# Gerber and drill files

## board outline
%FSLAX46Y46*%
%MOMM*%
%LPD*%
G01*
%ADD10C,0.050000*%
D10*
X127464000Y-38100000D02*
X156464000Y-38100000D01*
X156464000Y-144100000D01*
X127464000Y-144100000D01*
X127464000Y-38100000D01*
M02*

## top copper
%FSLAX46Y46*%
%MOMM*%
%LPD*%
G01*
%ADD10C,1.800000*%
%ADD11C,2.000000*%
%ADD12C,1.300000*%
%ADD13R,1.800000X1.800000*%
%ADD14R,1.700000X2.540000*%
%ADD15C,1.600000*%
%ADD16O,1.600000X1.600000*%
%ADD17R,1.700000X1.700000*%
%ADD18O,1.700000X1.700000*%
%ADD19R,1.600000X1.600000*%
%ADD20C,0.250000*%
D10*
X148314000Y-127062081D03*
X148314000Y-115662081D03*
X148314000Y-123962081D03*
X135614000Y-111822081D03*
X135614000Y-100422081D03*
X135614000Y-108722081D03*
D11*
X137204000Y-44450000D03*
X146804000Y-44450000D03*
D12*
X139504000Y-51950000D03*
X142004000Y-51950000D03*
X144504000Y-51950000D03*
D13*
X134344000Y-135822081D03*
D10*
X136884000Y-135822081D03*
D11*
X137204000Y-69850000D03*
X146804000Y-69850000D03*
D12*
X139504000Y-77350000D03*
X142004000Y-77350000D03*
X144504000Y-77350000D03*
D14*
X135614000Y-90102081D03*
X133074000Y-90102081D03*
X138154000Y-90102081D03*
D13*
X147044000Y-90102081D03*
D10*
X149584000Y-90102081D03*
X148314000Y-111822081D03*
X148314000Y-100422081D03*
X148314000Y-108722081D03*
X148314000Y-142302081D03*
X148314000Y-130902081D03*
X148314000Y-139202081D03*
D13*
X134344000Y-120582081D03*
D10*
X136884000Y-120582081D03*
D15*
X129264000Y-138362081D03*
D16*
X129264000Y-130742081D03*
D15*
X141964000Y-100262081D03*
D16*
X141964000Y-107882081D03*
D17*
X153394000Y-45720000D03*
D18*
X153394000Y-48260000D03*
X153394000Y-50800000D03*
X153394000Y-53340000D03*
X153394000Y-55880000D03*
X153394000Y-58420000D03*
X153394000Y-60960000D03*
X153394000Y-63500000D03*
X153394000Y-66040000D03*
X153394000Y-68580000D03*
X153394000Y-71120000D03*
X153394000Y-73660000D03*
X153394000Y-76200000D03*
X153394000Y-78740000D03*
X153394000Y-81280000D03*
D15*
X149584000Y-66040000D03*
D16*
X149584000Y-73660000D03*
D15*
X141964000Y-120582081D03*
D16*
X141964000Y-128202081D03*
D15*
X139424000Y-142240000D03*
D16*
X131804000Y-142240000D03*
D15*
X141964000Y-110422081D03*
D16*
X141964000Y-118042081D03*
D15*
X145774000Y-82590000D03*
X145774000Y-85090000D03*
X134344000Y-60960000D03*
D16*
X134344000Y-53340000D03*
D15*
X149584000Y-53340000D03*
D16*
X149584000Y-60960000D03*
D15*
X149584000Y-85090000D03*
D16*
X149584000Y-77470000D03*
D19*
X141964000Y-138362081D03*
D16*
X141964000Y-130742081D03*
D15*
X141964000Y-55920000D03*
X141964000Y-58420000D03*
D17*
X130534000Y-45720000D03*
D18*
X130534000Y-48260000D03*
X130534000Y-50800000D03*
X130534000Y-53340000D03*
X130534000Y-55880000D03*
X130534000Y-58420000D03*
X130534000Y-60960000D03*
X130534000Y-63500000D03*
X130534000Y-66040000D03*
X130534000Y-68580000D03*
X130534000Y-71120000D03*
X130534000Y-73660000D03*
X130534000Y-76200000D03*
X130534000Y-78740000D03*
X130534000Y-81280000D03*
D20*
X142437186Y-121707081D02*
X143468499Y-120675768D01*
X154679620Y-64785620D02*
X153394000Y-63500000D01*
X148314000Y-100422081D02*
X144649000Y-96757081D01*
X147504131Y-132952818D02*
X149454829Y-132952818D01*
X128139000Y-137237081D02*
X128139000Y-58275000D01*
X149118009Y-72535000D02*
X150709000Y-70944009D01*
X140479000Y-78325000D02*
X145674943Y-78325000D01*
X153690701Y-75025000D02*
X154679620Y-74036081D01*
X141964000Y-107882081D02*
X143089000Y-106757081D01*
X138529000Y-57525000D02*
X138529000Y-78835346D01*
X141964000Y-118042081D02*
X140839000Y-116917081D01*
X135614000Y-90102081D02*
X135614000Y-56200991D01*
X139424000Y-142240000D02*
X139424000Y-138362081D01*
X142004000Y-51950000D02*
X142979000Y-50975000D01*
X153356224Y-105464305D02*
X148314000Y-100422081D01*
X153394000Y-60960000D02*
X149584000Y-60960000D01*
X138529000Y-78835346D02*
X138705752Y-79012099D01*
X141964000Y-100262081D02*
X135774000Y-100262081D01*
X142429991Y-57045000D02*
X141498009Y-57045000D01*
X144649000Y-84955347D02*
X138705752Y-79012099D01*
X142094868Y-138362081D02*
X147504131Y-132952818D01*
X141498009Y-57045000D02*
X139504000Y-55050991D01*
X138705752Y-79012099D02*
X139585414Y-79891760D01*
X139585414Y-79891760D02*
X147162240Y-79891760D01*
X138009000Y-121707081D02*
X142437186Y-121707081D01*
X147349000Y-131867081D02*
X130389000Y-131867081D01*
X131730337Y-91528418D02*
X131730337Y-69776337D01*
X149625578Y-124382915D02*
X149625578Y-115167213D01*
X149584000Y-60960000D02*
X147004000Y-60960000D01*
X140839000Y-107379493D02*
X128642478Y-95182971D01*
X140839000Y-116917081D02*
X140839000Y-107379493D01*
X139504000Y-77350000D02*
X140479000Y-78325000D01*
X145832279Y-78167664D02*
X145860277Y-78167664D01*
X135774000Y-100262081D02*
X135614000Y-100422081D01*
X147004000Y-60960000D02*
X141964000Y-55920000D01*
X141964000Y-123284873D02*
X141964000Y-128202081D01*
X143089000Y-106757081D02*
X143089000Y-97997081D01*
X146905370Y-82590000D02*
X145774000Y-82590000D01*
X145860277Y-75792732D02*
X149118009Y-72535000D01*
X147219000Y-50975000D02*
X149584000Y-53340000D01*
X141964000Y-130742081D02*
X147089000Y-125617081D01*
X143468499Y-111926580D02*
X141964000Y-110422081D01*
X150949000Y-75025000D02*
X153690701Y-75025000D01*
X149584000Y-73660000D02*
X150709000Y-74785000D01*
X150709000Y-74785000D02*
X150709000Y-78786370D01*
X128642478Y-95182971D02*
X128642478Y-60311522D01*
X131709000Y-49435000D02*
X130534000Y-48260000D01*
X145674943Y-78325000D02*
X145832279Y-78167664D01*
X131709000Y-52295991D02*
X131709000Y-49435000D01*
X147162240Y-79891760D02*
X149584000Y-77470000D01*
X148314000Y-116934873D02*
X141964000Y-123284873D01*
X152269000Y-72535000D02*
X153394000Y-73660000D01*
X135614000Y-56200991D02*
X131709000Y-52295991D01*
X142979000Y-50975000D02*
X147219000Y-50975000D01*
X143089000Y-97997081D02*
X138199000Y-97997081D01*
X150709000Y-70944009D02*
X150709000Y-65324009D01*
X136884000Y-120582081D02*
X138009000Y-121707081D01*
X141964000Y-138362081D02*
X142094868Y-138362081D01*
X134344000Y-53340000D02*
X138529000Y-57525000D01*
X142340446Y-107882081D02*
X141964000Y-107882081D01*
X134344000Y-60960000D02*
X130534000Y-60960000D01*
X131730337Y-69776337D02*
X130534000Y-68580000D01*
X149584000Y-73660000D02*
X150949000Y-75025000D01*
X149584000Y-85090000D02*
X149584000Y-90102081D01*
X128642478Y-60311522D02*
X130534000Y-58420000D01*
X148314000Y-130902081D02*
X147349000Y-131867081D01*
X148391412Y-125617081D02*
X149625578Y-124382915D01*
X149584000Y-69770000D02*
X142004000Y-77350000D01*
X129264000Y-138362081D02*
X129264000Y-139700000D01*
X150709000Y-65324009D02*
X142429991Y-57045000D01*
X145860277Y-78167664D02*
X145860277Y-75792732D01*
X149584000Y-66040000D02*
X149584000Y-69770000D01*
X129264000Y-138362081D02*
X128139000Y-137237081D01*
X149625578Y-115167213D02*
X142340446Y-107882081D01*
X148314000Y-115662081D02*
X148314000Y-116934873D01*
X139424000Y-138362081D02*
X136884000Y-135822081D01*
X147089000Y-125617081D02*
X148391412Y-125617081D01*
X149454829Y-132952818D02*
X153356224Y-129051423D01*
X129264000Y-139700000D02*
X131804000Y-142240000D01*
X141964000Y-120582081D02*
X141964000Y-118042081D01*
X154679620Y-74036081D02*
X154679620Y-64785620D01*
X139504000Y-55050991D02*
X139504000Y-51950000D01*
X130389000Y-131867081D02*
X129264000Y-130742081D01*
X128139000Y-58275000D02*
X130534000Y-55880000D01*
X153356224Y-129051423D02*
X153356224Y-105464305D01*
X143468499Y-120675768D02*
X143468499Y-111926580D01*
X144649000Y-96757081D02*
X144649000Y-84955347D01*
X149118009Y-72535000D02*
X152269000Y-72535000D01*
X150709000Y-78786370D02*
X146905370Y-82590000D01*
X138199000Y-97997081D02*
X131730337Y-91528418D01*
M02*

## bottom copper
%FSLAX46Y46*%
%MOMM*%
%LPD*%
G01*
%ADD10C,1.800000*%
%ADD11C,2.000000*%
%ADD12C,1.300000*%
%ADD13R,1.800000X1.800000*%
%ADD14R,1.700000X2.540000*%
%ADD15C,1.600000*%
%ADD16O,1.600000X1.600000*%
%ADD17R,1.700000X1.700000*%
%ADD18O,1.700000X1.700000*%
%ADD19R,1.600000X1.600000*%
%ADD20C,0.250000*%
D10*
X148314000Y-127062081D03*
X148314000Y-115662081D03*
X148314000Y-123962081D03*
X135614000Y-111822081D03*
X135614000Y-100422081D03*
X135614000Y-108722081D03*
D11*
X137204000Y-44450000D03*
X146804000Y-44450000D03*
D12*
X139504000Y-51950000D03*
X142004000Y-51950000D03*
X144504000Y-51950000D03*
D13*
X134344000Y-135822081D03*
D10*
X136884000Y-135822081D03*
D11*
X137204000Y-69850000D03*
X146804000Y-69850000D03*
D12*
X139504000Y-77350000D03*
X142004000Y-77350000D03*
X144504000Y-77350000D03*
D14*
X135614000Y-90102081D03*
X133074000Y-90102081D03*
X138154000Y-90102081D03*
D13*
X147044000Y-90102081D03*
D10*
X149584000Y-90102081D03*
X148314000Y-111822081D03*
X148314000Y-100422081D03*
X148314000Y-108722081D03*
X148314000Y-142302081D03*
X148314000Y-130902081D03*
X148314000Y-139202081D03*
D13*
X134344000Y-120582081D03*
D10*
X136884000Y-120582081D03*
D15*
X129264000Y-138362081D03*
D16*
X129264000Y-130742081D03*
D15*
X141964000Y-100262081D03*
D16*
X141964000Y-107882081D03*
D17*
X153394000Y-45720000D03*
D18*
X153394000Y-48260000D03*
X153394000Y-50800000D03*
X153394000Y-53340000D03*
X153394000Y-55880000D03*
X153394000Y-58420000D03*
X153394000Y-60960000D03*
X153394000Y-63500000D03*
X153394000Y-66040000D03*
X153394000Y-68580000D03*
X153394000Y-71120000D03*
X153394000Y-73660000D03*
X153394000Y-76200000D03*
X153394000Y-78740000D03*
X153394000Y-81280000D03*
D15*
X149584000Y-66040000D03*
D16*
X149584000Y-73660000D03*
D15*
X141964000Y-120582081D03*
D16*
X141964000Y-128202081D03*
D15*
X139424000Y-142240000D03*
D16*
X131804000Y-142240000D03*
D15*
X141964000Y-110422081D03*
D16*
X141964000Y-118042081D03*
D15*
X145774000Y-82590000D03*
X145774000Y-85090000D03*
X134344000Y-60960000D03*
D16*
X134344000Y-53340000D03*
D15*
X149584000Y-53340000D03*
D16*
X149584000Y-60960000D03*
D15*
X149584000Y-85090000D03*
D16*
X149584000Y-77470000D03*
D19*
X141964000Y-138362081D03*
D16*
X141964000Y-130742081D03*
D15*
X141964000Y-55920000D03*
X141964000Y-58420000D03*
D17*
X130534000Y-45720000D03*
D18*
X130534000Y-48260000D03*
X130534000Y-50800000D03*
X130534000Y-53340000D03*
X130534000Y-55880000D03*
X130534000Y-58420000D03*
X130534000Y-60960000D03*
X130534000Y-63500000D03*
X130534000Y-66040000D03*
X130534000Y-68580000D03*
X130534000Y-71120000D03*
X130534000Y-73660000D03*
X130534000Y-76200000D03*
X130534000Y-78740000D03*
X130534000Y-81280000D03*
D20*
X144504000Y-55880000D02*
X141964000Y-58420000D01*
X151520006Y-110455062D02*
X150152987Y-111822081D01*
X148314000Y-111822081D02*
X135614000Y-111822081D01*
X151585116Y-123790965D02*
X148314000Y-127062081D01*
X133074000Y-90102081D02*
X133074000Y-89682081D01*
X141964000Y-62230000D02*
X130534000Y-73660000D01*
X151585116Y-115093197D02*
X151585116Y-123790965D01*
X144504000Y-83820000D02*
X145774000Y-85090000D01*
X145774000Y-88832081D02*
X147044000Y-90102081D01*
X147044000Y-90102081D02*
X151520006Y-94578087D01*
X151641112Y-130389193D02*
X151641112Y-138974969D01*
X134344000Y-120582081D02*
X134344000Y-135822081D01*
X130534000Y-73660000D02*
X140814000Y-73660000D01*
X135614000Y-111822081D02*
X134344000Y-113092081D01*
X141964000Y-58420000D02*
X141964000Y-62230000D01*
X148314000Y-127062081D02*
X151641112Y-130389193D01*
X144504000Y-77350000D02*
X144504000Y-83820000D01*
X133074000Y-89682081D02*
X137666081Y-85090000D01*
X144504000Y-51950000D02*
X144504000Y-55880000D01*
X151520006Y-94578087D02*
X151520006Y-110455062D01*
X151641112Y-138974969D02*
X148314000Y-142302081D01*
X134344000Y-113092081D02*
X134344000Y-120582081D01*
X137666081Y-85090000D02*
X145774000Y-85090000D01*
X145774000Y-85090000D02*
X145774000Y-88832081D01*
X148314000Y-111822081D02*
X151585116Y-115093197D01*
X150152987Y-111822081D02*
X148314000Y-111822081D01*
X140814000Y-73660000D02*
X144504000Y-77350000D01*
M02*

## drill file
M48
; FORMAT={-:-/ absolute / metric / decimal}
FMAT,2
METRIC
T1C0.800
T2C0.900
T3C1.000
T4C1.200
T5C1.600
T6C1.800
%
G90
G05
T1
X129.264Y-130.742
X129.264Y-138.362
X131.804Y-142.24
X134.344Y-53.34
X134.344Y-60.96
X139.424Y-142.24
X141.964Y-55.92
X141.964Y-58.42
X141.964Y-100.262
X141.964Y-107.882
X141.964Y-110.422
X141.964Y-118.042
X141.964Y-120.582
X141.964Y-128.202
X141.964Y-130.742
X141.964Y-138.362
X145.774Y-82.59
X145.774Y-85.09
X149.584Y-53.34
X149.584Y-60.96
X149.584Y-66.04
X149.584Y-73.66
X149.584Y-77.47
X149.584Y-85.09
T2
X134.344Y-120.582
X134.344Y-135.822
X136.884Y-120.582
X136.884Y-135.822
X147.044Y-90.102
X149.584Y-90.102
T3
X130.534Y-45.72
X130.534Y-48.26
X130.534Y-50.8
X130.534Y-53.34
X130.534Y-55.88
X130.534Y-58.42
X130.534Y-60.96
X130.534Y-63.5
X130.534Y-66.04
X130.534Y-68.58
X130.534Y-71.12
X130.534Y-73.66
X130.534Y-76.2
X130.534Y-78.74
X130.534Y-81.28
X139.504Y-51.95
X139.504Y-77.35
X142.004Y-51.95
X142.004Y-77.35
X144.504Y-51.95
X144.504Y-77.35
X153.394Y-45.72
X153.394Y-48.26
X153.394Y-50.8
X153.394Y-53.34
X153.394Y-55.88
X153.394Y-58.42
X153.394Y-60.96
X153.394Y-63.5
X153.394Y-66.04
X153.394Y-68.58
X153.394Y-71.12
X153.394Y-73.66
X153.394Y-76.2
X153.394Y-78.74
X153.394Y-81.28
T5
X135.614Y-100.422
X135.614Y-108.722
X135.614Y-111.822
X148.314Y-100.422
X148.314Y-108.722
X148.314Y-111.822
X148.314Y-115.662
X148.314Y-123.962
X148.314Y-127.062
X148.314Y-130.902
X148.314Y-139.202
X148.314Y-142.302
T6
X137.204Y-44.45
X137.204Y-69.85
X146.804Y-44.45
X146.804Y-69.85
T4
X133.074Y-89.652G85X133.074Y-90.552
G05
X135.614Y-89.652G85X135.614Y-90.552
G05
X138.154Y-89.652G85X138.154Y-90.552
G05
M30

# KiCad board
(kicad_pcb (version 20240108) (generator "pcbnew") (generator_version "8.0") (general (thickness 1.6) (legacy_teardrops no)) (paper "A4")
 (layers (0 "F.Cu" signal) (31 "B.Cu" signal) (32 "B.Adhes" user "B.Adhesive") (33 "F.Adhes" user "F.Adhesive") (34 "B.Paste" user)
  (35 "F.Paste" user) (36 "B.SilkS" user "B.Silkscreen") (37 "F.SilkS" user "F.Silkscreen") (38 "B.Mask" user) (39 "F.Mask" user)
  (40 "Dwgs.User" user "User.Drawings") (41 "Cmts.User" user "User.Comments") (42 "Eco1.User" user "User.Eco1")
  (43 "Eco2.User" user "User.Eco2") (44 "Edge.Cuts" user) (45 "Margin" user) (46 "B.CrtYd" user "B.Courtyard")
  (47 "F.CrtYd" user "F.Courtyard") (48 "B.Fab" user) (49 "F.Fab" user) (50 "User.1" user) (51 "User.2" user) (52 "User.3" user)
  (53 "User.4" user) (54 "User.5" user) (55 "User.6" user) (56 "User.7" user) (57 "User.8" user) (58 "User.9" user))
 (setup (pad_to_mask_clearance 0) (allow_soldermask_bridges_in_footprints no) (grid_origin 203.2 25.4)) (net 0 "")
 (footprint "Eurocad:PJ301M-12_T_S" (layer "F.Cu") (at 148.314 120.582081)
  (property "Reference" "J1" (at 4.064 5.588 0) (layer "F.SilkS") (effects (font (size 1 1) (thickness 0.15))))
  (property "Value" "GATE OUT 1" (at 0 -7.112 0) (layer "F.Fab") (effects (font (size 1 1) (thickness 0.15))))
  (pad "S" thru_hole circle (at 0 6.48) (size 1.8 1.8) (drill 1.6) (layers "*.Cu" "*.Mask" "F.SilkS") (remove_unused_layers no))
  (pad "T" thru_hole circle (at 0 -4.92) (size 1.8 1.8) (drill 1.6) (layers "*.Cu" "*.Mask" "F.SilkS") (remove_unused_layers no))
  (pad "TN" thru_hole circle (at 0 3.38) (size 1.8 1.8) (drill 1.6) (layers "*.Cu" "*.Mask" "F.SilkS") (remove_unused_layers no)))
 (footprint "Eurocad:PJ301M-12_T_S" (layer "F.Cu") (at 135.614 105.342081)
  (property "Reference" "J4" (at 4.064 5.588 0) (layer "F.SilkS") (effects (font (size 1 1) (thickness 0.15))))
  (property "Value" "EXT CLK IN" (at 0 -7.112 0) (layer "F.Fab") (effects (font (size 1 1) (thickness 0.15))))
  (pad "S" thru_hole circle (at 0 6.48) (size 1.8 1.8) (drill 1.6) (layers "*.Cu" "*.Mask" "F.SilkS") (remove_unused_layers no))
  (pad "T" thru_hole circle (at 0 -4.92) (size 1.8 1.8) (drill 1.6) (layers "*.Cu" "*.Mask" "F.SilkS") (remove_unused_layers no))
  (pad "TN" thru_hole circle (at 0 3.38) (size 1.8 1.8) (drill 1.6) (layers "*.Cu" "*.Mask" "F.SilkS") (remove_unused_layers no)))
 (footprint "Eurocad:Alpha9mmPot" (layer "F.Cu") (at 142.004 44.45)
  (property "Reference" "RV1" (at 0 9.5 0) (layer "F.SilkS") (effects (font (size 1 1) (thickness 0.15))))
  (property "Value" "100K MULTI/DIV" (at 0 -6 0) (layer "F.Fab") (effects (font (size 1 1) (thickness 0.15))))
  (pad "" thru_hole circle (at -4.8 0) (size 2 2) (drill 1.8) (layers "*.Cu" "*.Mask" "F.SilkS") (remove_unused_layers no))
  (pad "" thru_hole circle (at 4.8 0) (size 2 2) (drill 1.8) (layers "*.Cu" "*.Mask" "F.SilkS") (remove_unused_layers no))
  (pad "1" thru_hole circle (at -2.5 7.5) (size 1.3 1.3) (drill 1) (layers "*.Cu" "*.Mask" "F.SilkS") (remove_unused_layers no))
  (pad "2" thru_hole circle (at 0 7.5) (size 1.3 1.3) (drill 1) (layers "*.Cu" "*.Mask" "F.SilkS") (remove_unused_layers no))
  (pad "3" thru_hole circle (at 2.5 7.5) (size 1.3 1.3) (drill 1) (layers "*.Cu" "*.Mask" "F.SilkS") (remove_unused_layers no)))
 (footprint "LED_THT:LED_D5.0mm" (layer "F.Cu") (at 134.344 135.822081)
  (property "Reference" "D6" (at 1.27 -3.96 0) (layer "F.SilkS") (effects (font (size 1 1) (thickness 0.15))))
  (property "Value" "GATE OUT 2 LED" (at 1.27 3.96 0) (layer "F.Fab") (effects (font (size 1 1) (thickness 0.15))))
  (pad "1" thru_hole rect (at 0 0) (size 1.8 1.8) (drill 0.9) (layers "*.Cu" "*.Mask") (remove_unused_layers no))
  (pad "2" thru_hole circle (at 2.54 0) (size 1.8 1.8) (drill 0.9) (layers "*.Cu" "*.Mask") (remove_unused_layers no)))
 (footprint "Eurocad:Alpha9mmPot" (layer "F.Cu") (at 142.004 69.85)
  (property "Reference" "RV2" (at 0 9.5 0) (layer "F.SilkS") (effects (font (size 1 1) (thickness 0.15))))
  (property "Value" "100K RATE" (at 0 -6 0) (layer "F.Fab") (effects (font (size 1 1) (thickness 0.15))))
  (pad "" thru_hole circle (at -4.8 0) (size 2 2) (drill 1.8) (layers "*.Cu" "*.Mask" "F.SilkS") (remove_unused_layers no))
  (pad "" thru_hole circle (at 4.8 0) (size 2 2) (drill 1.8) (layers "*.Cu" "*.Mask" "F.SilkS") (remove_unused_layers no))
  (pad "1" thru_hole circle (at -2.5 7.5) (size 1.3 1.3) (drill 1) (layers "*.Cu" "*.Mask" "F.SilkS") (remove_unused_layers no))
  (pad "2" thru_hole circle (at 0 7.5) (size 1.3 1.3) (drill 1) (layers "*.Cu" "*.Mask" "F.SilkS") (remove_unused_layers no))
  (pad "3" thru_hole circle (at 2.5 7.5) (size 1.3 1.3) (drill 1) (layers "*.Cu" "*.Mask" "F.SilkS") (remove_unused_layers no)))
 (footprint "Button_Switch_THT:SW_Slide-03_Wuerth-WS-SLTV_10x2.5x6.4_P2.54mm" (layer "F.Cu") (at 135.614 90.102081)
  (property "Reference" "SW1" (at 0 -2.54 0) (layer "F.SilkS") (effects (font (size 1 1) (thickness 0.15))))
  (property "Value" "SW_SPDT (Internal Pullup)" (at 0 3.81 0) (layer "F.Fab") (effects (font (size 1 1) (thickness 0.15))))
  (pad "1" thru_hole rect (at 0 0) (size 1.7 2.54) (drill oval 1.2 2.1) (layers "*.Cu" "*.Mask") (remove_unused_layers no))
  (pad "2" thru_hole rect (at -2.54 0) (size 1.7 2.54) (drill oval 1.2 2.1) (layers "*.Cu" "*.Mask") (remove_unused_layers no))
  (pad "3" thru_hole rect (at 2.54 0) (size 1.7 2.54) (drill oval 1.2 2.1) (layers "*.Cu" "*.Mask") (remove_unused_layers no)))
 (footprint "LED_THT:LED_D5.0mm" (layer "F.Cu") (at 147.044 90.102081)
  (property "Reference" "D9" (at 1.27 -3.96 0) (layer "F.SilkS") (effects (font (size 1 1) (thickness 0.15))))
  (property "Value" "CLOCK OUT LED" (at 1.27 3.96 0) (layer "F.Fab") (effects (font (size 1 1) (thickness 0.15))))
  (pad "1" thru_hole rect (at 0 0) (size 1.8 1.8) (drill 0.9) (layers "*.Cu" "*.Mask") (remove_unused_layers no))
  (pad "2" thru_hole circle (at 2.54 0) (size 1.8 1.8) (drill 0.9) (layers "*.Cu" "*.Mask") (remove_unused_layers no)))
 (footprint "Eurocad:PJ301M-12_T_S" (layer "F.Cu") (at 148.314 105.342081)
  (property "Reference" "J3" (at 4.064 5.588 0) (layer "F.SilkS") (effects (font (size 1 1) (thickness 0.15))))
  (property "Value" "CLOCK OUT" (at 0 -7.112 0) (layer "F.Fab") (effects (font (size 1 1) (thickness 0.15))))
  (pad "S" thru_hole circle (at 0 6.48) (size 1.8 1.8) (drill 1.6) (layers "*.Cu" "*.Mask" "F.SilkS") (remove_unused_layers no))
  (pad "T" thru_hole circle (at 0 -4.92) (size 1.8 1.8) (drill 1.6) (layers "*.Cu" "*.Mask" "F.SilkS") (remove_unused_layers no))
  (pad "TN" thru_hole circle (at 0 3.38) (size 1.8 1.8) (drill 1.6) (layers "*.Cu" "*.Mask" "F.SilkS") (remove_unused_layers no)))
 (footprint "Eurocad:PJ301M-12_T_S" (layer "F.Cu") (at 148.314 135.822081)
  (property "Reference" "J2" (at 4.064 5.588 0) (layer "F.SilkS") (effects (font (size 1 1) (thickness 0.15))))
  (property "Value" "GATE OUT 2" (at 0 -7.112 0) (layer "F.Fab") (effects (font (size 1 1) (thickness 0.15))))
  (pad "S" thru_hole circle (at 0 6.48) (size 1.8 1.8) (drill 1.6) (layers "*.Cu" "*.Mask" "F.SilkS") (remove_unused_layers no))
  (pad "T" thru_hole circle (at 0 -4.92) (size 1.8 1.8) (drill 1.6) (layers "*.Cu" "*.Mask" "F.SilkS") (remove_unused_layers no))
  (pad "TN" thru_hole circle (at 0 3.38) (size 1.8 1.8) (drill 1.6) (layers "*.Cu" "*.Mask" "F.SilkS") (remove_unused_layers no)))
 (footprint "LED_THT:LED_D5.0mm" (layer "F.Cu") (at 134.344 120.582081)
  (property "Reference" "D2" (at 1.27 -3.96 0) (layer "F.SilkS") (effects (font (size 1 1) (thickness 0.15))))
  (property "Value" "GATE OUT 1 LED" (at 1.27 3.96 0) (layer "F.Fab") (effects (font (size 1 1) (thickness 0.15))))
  (pad "1" thru_hole rect (at 0 0) (size 1.8 1.8) (drill 0.9) (layers "*.Cu" "*.Mask") (remove_unused_layers no))
  (pad "2" thru_hole circle (at 2.54 0) (size 1.8 1.8) (drill 0.9) (layers "*.Cu" "*.Mask") (remove_unused_layers no)))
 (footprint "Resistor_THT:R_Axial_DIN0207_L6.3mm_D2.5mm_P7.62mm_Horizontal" (layer "B.Cu") (at 129.264 138.362081 90)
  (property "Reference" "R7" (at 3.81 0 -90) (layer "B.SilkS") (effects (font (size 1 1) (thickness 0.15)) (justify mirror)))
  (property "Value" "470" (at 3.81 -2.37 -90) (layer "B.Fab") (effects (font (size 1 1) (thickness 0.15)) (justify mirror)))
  (pad "1" thru_hole circle (at 0 0 90) (size 1.6 1.6) (drill 0.8) (layers "*.Cu" "*.Mask") (remove_unused_layers no))
  (pad "2" thru_hole oval (at 7.62 0 90) (size 1.6 1.6) (drill 0.8) (layers "*.Cu" "*.Mask") (remove_unused_layers no)))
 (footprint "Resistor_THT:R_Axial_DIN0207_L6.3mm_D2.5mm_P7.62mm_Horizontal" (layer "B.Cu") (at 141.964 100.262081 -90)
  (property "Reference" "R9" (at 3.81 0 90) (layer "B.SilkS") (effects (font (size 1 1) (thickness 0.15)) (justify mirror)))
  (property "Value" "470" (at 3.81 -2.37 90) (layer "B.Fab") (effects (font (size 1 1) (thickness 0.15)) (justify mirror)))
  (pad "1" thru_hole circle (at 0 0 270) (size 1.6 1.6) (drill 0.8) (layers "*.Cu" "*.Mask") (remove_unused_layers no))
  (pad "2" thru_hole oval (at 7.62 0 270) (size 1.6 1.6) (drill 0.8) (layers "*.Cu" "*.Mask") (remove_unused_layers no)))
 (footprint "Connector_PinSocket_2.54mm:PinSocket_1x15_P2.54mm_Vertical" (layer "B.Cu") (at 153.394 45.72 180)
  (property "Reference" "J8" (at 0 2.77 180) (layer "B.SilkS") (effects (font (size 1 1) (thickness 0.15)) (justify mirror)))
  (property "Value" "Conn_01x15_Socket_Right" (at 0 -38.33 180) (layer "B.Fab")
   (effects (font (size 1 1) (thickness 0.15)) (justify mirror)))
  (pad "1" thru_hole rect (at 0 0 180) (size 1.7 1.7) (drill 1) (layers "*.Cu" "*.Mask") (remove_unused_layers no))
  (pad "2" thru_hole oval (at 0 -2.54 180) (size 1.7 1.7) (drill 1) (layers "*.Cu" "*.Mask") (remove_unused_layers no))
  (pad "3" thru_hole oval (at 0 -5.08 180) (size 1.7 1.7) (drill 1) (layers "*.Cu" "*.Mask") (remove_unused_layers no))
  (pad "4" thru_hole oval (at 0 -7.62 180) (size 1.7 1.7) (drill 1) (layers "*.Cu" "*.Mask") (remove_unused_layers no))
  (pad "5" thru_hole oval (at 0 -10.16 180) (size 1.7 1.7) (drill 1) (layers "*.Cu" "*.Mask") (remove_unused_layers no))
  (pad "6" thru_hole oval (at 0 -12.7 180) (size 1.7 1.7) (drill 1) (layers "*.Cu" "*.Mask") (remove_unused_layers no))
  (pad "7" thru_hole oval (at 0 -15.24 180) (size 1.7 1.7) (drill 1) (layers "*.Cu" "*.Mask") (remove_unused_layers no))
  (pad "8" thru_hole oval (at 0 -17.78 180) (size 1.7 1.7) (drill 1) (layers "*.Cu" "*.Mask") (remove_unused_layers no))
  (pad "9" thru_hole oval (at 0 -20.32 180) (size 1.7 1.7) (drill 1) (layers "*.Cu" "*.Mask") (remove_unused_layers no))
  (pad "10" thru_hole oval (at 0 -22.86 180) (size 1.7 1.7) (drill 1) (layers "*.Cu" "*.Mask") (remove_unused_layers no))
  (pad "11" thru_hole oval (at 0 -25.4 180) (size 1.7 1.7) (drill 1) (layers "*.Cu" "*.Mask") (remove_unused_layers no))
  (pad "12" thru_hole oval (at 0 -27.94 180) (size 1.7 1.7) (drill 1) (layers "*.Cu" "*.Mask") (remove_unused_layers no))
  (pad "13" thru_hole oval (at 0 -30.48 180) (size 1.7 1.7) (drill 1) (layers "*.Cu" "*.Mask") (remove_unused_layers no))
  (pad "14" thru_hole oval (at 0 -33.02 180) (size 1.7 1.7) (drill 1) (layers "*.Cu" "*.Mask") (remove_unused_layers no))
  (pad "15" thru_hole oval (at 0 -35.56 180) (size 1.7 1.7) (drill 1) (layers "*.Cu" "*.Mask") (remove_unused_layers no)))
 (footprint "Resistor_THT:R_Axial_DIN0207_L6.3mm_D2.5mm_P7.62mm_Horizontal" (layer "B.Cu") (at 149.584 66.04 -90)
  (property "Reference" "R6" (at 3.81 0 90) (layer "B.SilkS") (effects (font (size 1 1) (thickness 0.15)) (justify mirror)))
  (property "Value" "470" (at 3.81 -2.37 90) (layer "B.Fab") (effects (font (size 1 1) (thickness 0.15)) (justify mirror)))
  (pad "1" thru_hole circle (at 0 0 270) (size 1.6 1.6) (drill 0.8) (layers "*.Cu" "*.Mask") (remove_unused_layers no))
  (pad "2" thru_hole oval (at 7.62 0 270) (size 1.6 1.6) (drill 0.8) (layers "*.Cu" "*.Mask") (remove_unused_layers no)))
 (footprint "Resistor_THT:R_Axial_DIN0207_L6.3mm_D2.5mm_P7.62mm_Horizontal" (layer "B.Cu") (at 141.964 120.582081 -90)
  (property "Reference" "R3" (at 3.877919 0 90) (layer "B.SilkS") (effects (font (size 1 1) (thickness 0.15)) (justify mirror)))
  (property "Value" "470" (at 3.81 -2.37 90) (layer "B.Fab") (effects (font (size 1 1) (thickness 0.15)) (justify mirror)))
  (pad "1" thru_hole circle (at 0 0 270) (size 1.6 1.6) (drill 0.8) (layers "*.Cu" "*.Mask") (remove_unused_layers no))
  (pad "2" thru_hole oval (at 7.62 0 270) (size 1.6 1.6) (drill 0.8) (layers "*.Cu" "*.Mask") (remove_unused_layers no)))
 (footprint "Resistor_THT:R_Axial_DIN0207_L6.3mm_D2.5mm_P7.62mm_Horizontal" (layer "B.Cu") (at 139.424 142.24 180)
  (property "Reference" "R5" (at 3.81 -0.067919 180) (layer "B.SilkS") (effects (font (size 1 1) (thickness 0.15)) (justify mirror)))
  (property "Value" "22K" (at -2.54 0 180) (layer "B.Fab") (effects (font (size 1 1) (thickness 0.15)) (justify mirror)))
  (pad "1" thru_hole circle (at 0 0 180) (size 1.6 1.6) (drill 0.8) (layers "*.Cu" "*.Mask") (remove_unused_layers no))
  (pad "2" thru_hole oval (at 7.62 0 180) (size 1.6 1.6) (drill 0.8) (layers "*.Cu" "*.Mask") (remove_unused_layers no)))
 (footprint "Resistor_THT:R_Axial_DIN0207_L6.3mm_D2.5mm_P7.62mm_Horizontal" (layer "B.Cu") (at 141.964 110.422081 -90)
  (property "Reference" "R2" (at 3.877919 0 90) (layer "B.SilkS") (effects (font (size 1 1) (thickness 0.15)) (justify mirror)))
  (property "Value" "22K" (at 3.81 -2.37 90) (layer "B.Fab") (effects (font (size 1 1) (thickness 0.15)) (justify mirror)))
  (pad "1" thru_hole circle (at 0 0 270) (size 1.6 1.6) (drill 0.8) (layers "*.Cu" "*.Mask") (remove_unused_layers no))
  (pad "2" thru_hole oval (at 7.62 0 270) (size 1.6 1.6) (drill 0.8) (layers "*.Cu" "*.Mask") (remove_unused_layers no)))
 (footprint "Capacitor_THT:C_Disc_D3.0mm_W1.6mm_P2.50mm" (layer "B.Cu") (at 145.774 82.59 -90)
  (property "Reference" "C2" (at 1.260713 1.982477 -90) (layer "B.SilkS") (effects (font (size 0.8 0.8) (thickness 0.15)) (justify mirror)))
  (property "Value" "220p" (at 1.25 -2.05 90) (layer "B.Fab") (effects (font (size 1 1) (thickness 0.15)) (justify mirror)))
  (pad "1" thru_hole circle (at 0 0 270) (size 1.6 1.6) (drill 0.8) (layers "*.Cu" "*.Mask") (remove_unused_layers no))
  (pad "2" thru_hole circle (at 2.5 0 270) (size 1.6 1.6) (drill 0.8) (layers "*.Cu" "*.Mask") (remove_unused_layers no)))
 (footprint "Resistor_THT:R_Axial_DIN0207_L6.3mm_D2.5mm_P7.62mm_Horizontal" (layer "B.Cu") (at 134.344 60.96 90)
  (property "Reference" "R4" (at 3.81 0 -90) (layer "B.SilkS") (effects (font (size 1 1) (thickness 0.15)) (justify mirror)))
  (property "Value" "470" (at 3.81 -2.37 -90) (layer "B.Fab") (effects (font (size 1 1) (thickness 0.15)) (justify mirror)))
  (pad "1" thru_hole circle (at 0 0 90) (size 1.6 1.6) (drill 0.8) (layers "*.Cu" "*.Mask") (remove_unused_layers no))
  (pad "2" thru_hole oval (at 7.62 0 90) (size 1.6 1.6) (drill 0.8) (layers "*.Cu" "*.Mask") (remove_unused_layers no)))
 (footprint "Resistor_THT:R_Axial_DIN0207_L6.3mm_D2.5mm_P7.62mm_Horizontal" (layer "B.Cu") (at 149.584 53.34 -90)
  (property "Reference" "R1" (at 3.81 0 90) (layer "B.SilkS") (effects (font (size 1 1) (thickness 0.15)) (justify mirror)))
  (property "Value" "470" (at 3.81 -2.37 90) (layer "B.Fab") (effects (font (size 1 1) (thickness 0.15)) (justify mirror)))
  (pad "1" thru_hole circle (at 0 0 270) (size 1.6 1.6) (drill 0.8) (layers "*.Cu" "*.Mask") (remove_unused_layers no))
  (pad "2" thru_hole oval (at 7.62 0 270) (size 1.6 1.6) (drill 0.8) (layers "*.Cu" "*.Mask") (remove_unused_layers no)))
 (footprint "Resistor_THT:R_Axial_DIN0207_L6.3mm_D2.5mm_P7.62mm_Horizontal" (layer "B.Cu") (at 149.584 85.09 90)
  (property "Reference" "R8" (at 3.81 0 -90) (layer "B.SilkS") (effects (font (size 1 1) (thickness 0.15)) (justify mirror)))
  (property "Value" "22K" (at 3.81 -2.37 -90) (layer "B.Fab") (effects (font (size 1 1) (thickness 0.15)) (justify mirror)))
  (pad "1" thru_hole circle (at 0 0 90) (size 1.6 1.6) (drill 0.8) (layers "*.Cu" "*.Mask") (remove_unused_layers no))
  (pad "2" thru_hole oval (at 7.62 0 90) (size 1.6 1.6) (drill 0.8) (layers "*.Cu" "*.Mask") (remove_unused_layers no)))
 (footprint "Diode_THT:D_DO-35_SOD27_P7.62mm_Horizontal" (layer "B.Cu") (at 141.964 138.362081 90)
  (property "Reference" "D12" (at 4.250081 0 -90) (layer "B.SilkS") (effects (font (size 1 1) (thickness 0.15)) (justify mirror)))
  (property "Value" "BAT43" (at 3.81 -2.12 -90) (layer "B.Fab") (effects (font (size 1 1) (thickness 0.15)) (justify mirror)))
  (pad "1" thru_hole rect (at 0 0 90) (size 1.6 1.6) (drill 0.8) (layers "*.Cu" "*.Mask") (remove_unused_layers no))
  (pad "2" thru_hole oval (at 7.62 0 90) (size 1.6 1.6) (drill 0.8) (layers "*.Cu" "*.Mask") (remove_unused_layers no)))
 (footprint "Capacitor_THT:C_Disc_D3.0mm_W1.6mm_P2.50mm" (layer "B.Cu") (at 141.964 55.92 -90)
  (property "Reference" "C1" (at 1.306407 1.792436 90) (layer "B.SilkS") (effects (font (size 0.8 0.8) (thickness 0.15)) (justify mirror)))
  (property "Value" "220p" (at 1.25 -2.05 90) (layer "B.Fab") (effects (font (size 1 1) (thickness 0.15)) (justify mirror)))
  (pad "1" thru_hole circle (at 0 0 270) (size 1.6 1.6) (drill 0.8) (layers "*.Cu" "*.Mask") (remove_unused_layers no))
  (pad "2" thru_hole circle (at 2.5 0 270) (size 1.6 1.6) (drill 0.8) (layers "*.Cu" "*.Mask") (remove_unused_layers no)))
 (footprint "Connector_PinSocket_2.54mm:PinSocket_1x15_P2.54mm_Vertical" (layer "B.Cu") (at 130.534 45.72 180)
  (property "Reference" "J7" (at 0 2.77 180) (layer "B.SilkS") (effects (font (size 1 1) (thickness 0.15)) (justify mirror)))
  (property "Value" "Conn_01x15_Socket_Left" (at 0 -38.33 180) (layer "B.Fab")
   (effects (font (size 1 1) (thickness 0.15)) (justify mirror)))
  (pad "1" thru_hole rect (at 0 0 180) (size 1.7 1.7) (drill 1) (layers "*.Cu" "*.Mask") (remove_unused_layers no))
  (pad "2" thru_hole oval (at 0 -2.54 180) (size 1.7 1.7) (drill 1) (layers "*.Cu" "*.Mask") (remove_unused_layers no))
  (pad "3" thru_hole oval (at 0 -5.08 180) (size 1.7 1.7) (drill 1) (layers "*.Cu" "*.Mask") (remove_unused_layers no))
  (pad "4" thru_hole oval (at 0 -7.62 180) (size 1.7 1.7) (drill 1) (layers "*.Cu" "*.Mask") (remove_unused_layers no))
  (pad "5" thru_hole oval (at 0 -10.16 180) (size 1.7 1.7) (drill 1) (layers "*.Cu" "*.Mask") (remove_unused_layers no))
  (pad "6" thru_hole oval (at 0 -12.7 180) (size 1.7 1.7) (drill 1) (layers "*.Cu" "*.Mask") (remove_unused_layers no))
  (pad "7" thru_hole oval (at 0 -15.24 180) (size 1.7 1.7) (drill 1) (layers "*.Cu" "*.Mask") (remove_unused_layers no))
  (pad "8" thru_hole oval (at 0 -17.78 180) (size 1.7 1.7) (drill 1) (layers "*.Cu" "*.Mask") (remove_unused_layers no))
  (pad "9" thru_hole oval (at 0 -20.32 180) (size 1.7 1.7) (drill 1) (layers "*.Cu" "*.Mask") (remove_unused_layers no))
  (pad "10" thru_hole oval (at 0 -22.86 180) (size 1.7 1.7) (drill 1) (layers "*.Cu" "*.Mask") (remove_unused_layers no))
  (pad "11" thru_hole oval (at 0 -25.4 180) (size 1.7 1.7) (drill 1) (layers "*.Cu" "*.Mask") (remove_unused_layers no))
  (pad "12" thru_hole oval (at 0 -27.94 180) (size 1.7 1.7) (drill 1) (layers "*.Cu" "*.Mask") (remove_unused_layers no))
  (pad "13" thru_hole oval (at 0 -30.48 180) (size 1.7 1.7) (drill 1) (layers "*.Cu" "*.Mask") (remove_unused_layers no))
  (pad "14" thru_hole oval (at 0 -33.02 180) (size 1.7 1.7) (drill 1) (layers "*.Cu" "*.Mask") (remove_unused_layers no))
  (pad "15" thru_hole oval (at 0 -35.56 180) (size 1.7 1.7) (drill 1) (layers "*.Cu" "*.Mask") (remove_unused_layers no)))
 (gr_rect (start 127.464 38.1) (end 156.464 144.1) (stroke (width 0.05) (type default)) (fill none) (layer "Edge.Cuts"))
 (segment (start 142.437186 121.707081) (end 143.468499 120.675768) (width 0.25) (layer "F.Cu") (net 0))
 (segment (start 154.67962 64.78562) (end 153.394 63.5) (width 0.25) (layer "F.Cu") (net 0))
 (segment (start 148.314 100.422081) (end 144.649 96.757081) (width 0.25) (layer "F.Cu") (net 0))
 (segment (start 147.504131 132.952818) (end 149.454829 132.952818) (width 0.25) (layer "F.Cu") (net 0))
 (segment (start 128.139 137.237081) (end 128.139 58.275) (width 0.25) (layer "F.Cu") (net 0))
 (segment (start 149.118009 72.535) (end 150.709 70.944009) (width 0.25) (layer "F.Cu") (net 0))
 (segment (start 140.479 78.325) (end 145.674943 78.325) (width 0.25) (layer "F.Cu") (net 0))
 (segment (start 153.690701 75.025) (end 154.67962 74.036081) (width 0.25) (layer "F.Cu") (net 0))
 (segment (start 141.964 107.882081) (end 143.089 106.757081) (width 0.25) (layer "F.Cu") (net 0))
 (segment (start 138.529 57.525) (end 138.529 78.835346) (width 0.25) (layer "F.Cu") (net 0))
 (segment (start 141.964 118.042081) (end 140.839 116.917081) (width 0.25) (layer "F.Cu") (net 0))
 (segment (start 135.614 90.102081) (end 135.614 56.200991) (width 0.25) (layer "F.Cu") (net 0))
 (segment (start 139.424 142.24) (end 139.424 138.362081) (width 0.25) (layer "F.Cu") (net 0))
 (segment (start 142.004 51.95) (end 142.979 50.975) (width 0.25) (layer "F.Cu") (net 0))
 (segment (start 153.356224 105.464305) (end 148.314 100.422081) (width 0.25) (layer "F.Cu") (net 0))
 (segment (start 153.394 60.96) (end 149.584 60.96) (width 0.25) (layer "F.Cu") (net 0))
 (segment (start 138.529 78.835346) (end 138.705752 79.012099) (width 0.25) (layer "F.Cu") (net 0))
 (segment (start 141.964 100.262081) (end 135.774 100.262081) (width 0.25) (layer "F.Cu") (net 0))
 (segment (start 142.429991 57.045) (end 141.498009 57.045) (width 0.25) (layer "F.Cu") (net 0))
 (segment (start 144.649 84.955347) (end 138.705752 79.012099) (width 0.25) (layer "F.Cu") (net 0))
 (segment (start 142.094868 138.362081) (end 147.504131 132.952818) (width 0.25) (layer "F.Cu") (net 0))
 (segment (start 141.498009 57.045) (end 139.504 55.050991) (width 0.25) (layer "F.Cu") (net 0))
 (segment (start 138.705752 79.012099) (end 139.585414 79.89176) (width 0.25) (layer "F.Cu") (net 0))
 (segment (start 139.585414 79.89176) (end 147.16224 79.89176) (width 0.25) (layer "F.Cu") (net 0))
 (segment (start 138.009 121.707081) (end 142.437186 121.707081) (width 0.25) (layer "F.Cu") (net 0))
 (segment (start 147.349 131.867081) (end 130.389 131.867081) (width 0.25) (layer "F.Cu") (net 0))
 (segment (start 131.730337 91.528418) (end 131.730337 69.776337) (width 0.25) (layer "F.Cu") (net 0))
 (segment (start 149.625578 124.382915) (end 149.625578 115.167213) (width 0.25) (layer "F.Cu") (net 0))
 (segment (start 149.584 60.96) (end 147.004 60.96) (width 0.25) (layer "F.Cu") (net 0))
 (segment (start 140.839 107.379493) (end 128.642478 95.182971) (width 0.25) (layer "F.Cu") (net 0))
 (segment (start 140.839 116.917081) (end 140.839 107.379493) (width 0.25) (layer "F.Cu") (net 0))
 (segment (start 139.504 77.35) (end 140.479 78.325) (width 0.25) (layer "F.Cu") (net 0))
 (segment (start 145.832279 78.167664) (end 145.860277 78.167664) (width 0.25) (layer "F.Cu") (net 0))
 (segment (start 135.774 100.262081) (end 135.614 100.422081) (width 0.25) (layer "F.Cu") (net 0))
 (segment (start 147.004 60.96) (end 141.964 55.92) (width 0.25) (layer "F.Cu") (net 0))
 (segment (start 141.964 123.284873) (end 141.964 128.202081) (width 0.25) (layer "F.Cu") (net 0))
 (segment (start 143.089 106.757081) (end 143.089 97.997081) (width 0.25) (layer "F.Cu") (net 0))
 (segment (start 146.90537 82.59) (end 145.774 82.59) (width 0.25) (layer "F.Cu") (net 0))
 (segment (start 145.860277 75.792732) (end 149.118009 72.535) (width 0.25) (layer "F.Cu") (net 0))
 (segment (start 147.219 50.975) (end 149.584 53.34) (width 0.25) (layer "F.Cu") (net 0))
 (segment (start 141.964 130.742081) (end 147.089 125.617081) (width 0.25) (layer "F.Cu") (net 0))
 (segment (start 143.468499 111.92658) (end 141.964 110.422081) (width 0.25) (layer "F.Cu") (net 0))
 (segment (start 150.949 75.025) (end 153.690701 75.025) (width 0.25) (layer "F.Cu") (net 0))
 (segment (start 149.584 73.66) (end 150.709 74.785) (width 0.25) (layer "F.Cu") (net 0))
 (segment (start 150.709 74.785) (end 150.709 78.78637) (width 0.25) (layer "F.Cu") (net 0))
 (segment (start 128.642478 95.182971) (end 128.642478 60.311522) (width 0.25) (layer "F.Cu") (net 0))
 (segment (start 131.709 49.435) (end 130.534 48.26) (width 0.25) (layer "F.Cu") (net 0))
 (segment (start 145.674943 78.325) (end 145.832279 78.167664) (width 0.25) (layer "F.Cu") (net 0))
 (segment (start 131.709 52.295991) (end 131.709 49.435) (width 0.25) (layer "F.Cu") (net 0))
 (segment (start 147.16224 79.89176) (end 149.584 77.47) (width 0.25) (layer "F.Cu") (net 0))
 (segment (start 148.314 116.934873) (end 141.964 123.284873) (width 0.25) (layer "F.Cu") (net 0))
 (segment (start 152.269 72.535) (end 153.394 73.66) (width 0.25) (layer "F.Cu") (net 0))
 (segment (start 135.614 56.200991) (end 131.709 52.295991) (width 0.25) (layer "F.Cu") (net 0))
 (segment (start 142.979 50.975) (end 147.219 50.975) (width 0.25) (layer "F.Cu") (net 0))
 (segment (start 143.089 97.997081) (end 138.199 97.997081) (width 0.25) (layer "F.Cu") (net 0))
 (segment (start 150.709 70.944009) (end 150.709 65.324009) (width 0.25) (layer "F.Cu") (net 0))
 (segment (start 136.884 120.582081) (end 138.009 121.707081) (width 0.25) (layer "F.Cu") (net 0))
 (segment (start 141.964 138.362081) (end 142.094868 138.362081) (width 0.25) (layer "F.Cu") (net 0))
 (segment (start 134.344 53.34) (end 138.529 57.525) (width 0.25) (layer "F.Cu") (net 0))
 (segment (start 142.340446 107.882081) (end 141.964 107.882081) (width 0.25) (layer "F.Cu") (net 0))
 (segment (start 134.344 60.96) (end 130.534 60.96) (width 0.25) (layer "F.Cu") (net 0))
 (segment (start 131.730337 69.776337) (end 130.534 68.58) (width 0.25) (layer "F.Cu") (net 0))
 (segment (start 149.584 73.66) (end 150.949 75.025) (width 0.25) (layer "F.Cu") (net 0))
 (segment (start 149.584 85.09) (end 149.584 90.102081) (width 0.25) (layer "F.Cu") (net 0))
 (segment (start 128.642478 60.311522) (end 130.534 58.42) (width 0.25) (layer "F.Cu") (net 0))
 (segment (start 148.314 130.902081) (end 147.349 131.867081) (width 0.25) (layer "F.Cu") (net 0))
 (segment (start 148.391412 125.617081) (end 149.625578 124.382915) (width 0.25) (layer "F.Cu") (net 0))
 (segment (start 149.584 69.77) (end 142.004 77.35) (width 0.25) (layer "F.Cu") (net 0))
 (segment (start 129.264 138.362081) (end 129.264 139.7) (width 0.25) (layer "F.Cu") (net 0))
 (segment (start 150.709 65.324009) (end 142.429991 57.045) (width 0.25) (layer "F.Cu") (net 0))
 (segment (start 145.860277 78.167664) (end 145.860277 75.792732) (width 0.25) (layer "F.Cu") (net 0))
 (segment (start 149.584 66.04) (end 149.584 69.77) (width 0.25) (layer "F.Cu") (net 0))
 (segment (start 129.264 138.362081) (end 128.139 137.237081) (width 0.25) (layer "F.Cu") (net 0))
 (segment (start 149.625578 115.167213) (end 142.340446 107.882081) (width 0.25) (layer "F.Cu") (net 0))
 (segment (start 148.314 115.662081) (end 148.314 116.934873) (width 0.25) (layer "F.Cu") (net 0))
 (segment (start 139.424 138.362081) (end 136.884 135.822081) (width 0.25) (layer "F.Cu") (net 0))
 (segment (start 147.089 125.617081) (end 148.391412 125.617081) (width 0.25) (layer "F.Cu") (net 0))
 (segment (start 149.454829 132.952818) (end 153.356224 129.051423) (width 0.25) (layer "F.Cu") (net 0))
 (segment (start 129.264 139.7) (end 131.804 142.24) (width 0.25) (layer "F.Cu") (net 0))
 (segment (start 141.964 120.582081) (end 141.964 118.042081) (width 0.25) (layer "F.Cu") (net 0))
 (segment (start 154.67962 74.036081) (end 154.67962 64.78562) (width 0.25) (layer "F.Cu") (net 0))
 (segment (start 139.504 55.050991) (end 139.504 51.95) (width 0.25) (layer "F.Cu") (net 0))
 (segment (start 130.389 131.867081) (end 129.264 130.742081) (width 0.25) (layer "F.Cu") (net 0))
 (segment (start 128.139 58.275) (end 130.534 55.88) (width 0.25) (layer "F.Cu") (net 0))
 (segment (start 153.356224 129.051423) (end 153.356224 105.464305) (width 0.25) (layer "F.Cu") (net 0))
 (segment (start 143.468499 120.675768) (end 143.468499 111.92658) (width 0.25) (layer "F.Cu") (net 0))
 (segment (start 144.649 96.757081) (end 144.649 84.955347) (width 0.25) (layer "F.Cu") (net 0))
 (segment (start 149.118009 72.535) (end 152.269 72.535) (width 0.25) (layer "F.Cu") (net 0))
 (segment (start 150.709 78.78637) (end 146.90537 82.59) (width 0.25) (layer "F.Cu") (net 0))
 (segment (start 138.199 97.997081) (end 131.730337 91.528418) (width 0.25) (layer "F.Cu") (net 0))
 (segment (start 144.504 55.88) (end 141.964 58.42) (width 0.25) (layer "B.Cu") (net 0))
 (segment (start 151.520006 110.455062) (end 150.152987 111.822081) (width 0.25) (layer "B.Cu") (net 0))
 (segment (start 148.314 111.822081) (end 135.614 111.822081) (width 0.25) (layer "B.Cu") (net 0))
 (segment (start 151.585116 123.790965) (end 148.314 127.062081) (width 0.25) (layer "B.Cu") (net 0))
 (segment (start 133.074 90.102081) (end 133.074 89.682081) (width 0.25) (layer "B.Cu") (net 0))
 (segment (start 141.964 62.23) (end 130.534 73.66) (width 0.25) (layer "B.Cu") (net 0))
 (segment (start 151.585116 115.093197) (end 151.585116 123.790965) (width 0.25) (layer "B.Cu") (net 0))
 (segment (start 144.504 83.82) (end 145.774 85.09) (width 0.25) (layer "B.Cu") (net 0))
 (segment (start 145.774 88.832081) (end 147.044 90.102081) (width 0.25) (layer "B.Cu") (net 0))
 (segment (start 147.044 90.102081) (end 151.520006 94.578087) (width 0.25) (layer "B.Cu") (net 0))
 (segment (start 151.641112 130.389193) (end 151.641112 138.974969) (width 0.25) (layer "B.Cu") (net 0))
 (segment (start 134.344 120.582081) (end 134.344 135.822081) (width 0.25) (layer "B.Cu") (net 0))
 (segment (start 130.534 73.66) (end 140.814 73.66) (width 0.25) (layer "B.Cu") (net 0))
 (segment (start 135.614 111.822081) (end 134.344 113.092081) (width 0.25) (layer "B.Cu") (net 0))
 (segment (start 141.964 58.42) (end 141.964 62.23) (width 0.25) (layer "B.Cu") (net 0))
 (segment (start 148.314 127.062081) (end 151.641112 130.389193) (width 0.25) (layer "B.Cu") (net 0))
 (segment (start 144.504 77.35) (end 144.504 83.82) (width 0.25) (layer "B.Cu") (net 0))
 (segment (start 133.074 89.682081) (end 137.666081 85.09) (width 0.25) (layer "B.Cu") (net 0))
 (segment (start 144.504 51.95) (end 144.504 55.88) (width 0.25) (layer "B.Cu") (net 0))
 (segment (start 151.520006 94.578087) (end 151.520006 110.455062) (width 0.25) (layer "B.Cu") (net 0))
 (segment (start 151.641112 138.974969) (end 148.314 142.302081) (width 0.25) (layer "B.Cu") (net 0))
 (segment (start 134.344 113.092081) (end 134.344 120.582081) (width 0.25) (layer "B.Cu") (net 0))
 (segment (start 137.666081 85.09) (end 145.774 85.09) (width 0.25) (layer "B.Cu") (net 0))
 (segment (start 145.774 85.09) (end 145.774 88.832081) (width 0.25) (layer "B.Cu") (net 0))
 (segment (start 148.314 111.822081) (end 151.585116 115.093197) (width 0.25) (layer "B.Cu") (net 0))
 (segment (start 150.152987 111.822081) (end 148.314 111.822081) (width 0.25) (layer "B.Cu") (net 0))
 (segment (start 140.814 73.66) (end 144.504 77.35) (width 0.25) (layer "B.Cu") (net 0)))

